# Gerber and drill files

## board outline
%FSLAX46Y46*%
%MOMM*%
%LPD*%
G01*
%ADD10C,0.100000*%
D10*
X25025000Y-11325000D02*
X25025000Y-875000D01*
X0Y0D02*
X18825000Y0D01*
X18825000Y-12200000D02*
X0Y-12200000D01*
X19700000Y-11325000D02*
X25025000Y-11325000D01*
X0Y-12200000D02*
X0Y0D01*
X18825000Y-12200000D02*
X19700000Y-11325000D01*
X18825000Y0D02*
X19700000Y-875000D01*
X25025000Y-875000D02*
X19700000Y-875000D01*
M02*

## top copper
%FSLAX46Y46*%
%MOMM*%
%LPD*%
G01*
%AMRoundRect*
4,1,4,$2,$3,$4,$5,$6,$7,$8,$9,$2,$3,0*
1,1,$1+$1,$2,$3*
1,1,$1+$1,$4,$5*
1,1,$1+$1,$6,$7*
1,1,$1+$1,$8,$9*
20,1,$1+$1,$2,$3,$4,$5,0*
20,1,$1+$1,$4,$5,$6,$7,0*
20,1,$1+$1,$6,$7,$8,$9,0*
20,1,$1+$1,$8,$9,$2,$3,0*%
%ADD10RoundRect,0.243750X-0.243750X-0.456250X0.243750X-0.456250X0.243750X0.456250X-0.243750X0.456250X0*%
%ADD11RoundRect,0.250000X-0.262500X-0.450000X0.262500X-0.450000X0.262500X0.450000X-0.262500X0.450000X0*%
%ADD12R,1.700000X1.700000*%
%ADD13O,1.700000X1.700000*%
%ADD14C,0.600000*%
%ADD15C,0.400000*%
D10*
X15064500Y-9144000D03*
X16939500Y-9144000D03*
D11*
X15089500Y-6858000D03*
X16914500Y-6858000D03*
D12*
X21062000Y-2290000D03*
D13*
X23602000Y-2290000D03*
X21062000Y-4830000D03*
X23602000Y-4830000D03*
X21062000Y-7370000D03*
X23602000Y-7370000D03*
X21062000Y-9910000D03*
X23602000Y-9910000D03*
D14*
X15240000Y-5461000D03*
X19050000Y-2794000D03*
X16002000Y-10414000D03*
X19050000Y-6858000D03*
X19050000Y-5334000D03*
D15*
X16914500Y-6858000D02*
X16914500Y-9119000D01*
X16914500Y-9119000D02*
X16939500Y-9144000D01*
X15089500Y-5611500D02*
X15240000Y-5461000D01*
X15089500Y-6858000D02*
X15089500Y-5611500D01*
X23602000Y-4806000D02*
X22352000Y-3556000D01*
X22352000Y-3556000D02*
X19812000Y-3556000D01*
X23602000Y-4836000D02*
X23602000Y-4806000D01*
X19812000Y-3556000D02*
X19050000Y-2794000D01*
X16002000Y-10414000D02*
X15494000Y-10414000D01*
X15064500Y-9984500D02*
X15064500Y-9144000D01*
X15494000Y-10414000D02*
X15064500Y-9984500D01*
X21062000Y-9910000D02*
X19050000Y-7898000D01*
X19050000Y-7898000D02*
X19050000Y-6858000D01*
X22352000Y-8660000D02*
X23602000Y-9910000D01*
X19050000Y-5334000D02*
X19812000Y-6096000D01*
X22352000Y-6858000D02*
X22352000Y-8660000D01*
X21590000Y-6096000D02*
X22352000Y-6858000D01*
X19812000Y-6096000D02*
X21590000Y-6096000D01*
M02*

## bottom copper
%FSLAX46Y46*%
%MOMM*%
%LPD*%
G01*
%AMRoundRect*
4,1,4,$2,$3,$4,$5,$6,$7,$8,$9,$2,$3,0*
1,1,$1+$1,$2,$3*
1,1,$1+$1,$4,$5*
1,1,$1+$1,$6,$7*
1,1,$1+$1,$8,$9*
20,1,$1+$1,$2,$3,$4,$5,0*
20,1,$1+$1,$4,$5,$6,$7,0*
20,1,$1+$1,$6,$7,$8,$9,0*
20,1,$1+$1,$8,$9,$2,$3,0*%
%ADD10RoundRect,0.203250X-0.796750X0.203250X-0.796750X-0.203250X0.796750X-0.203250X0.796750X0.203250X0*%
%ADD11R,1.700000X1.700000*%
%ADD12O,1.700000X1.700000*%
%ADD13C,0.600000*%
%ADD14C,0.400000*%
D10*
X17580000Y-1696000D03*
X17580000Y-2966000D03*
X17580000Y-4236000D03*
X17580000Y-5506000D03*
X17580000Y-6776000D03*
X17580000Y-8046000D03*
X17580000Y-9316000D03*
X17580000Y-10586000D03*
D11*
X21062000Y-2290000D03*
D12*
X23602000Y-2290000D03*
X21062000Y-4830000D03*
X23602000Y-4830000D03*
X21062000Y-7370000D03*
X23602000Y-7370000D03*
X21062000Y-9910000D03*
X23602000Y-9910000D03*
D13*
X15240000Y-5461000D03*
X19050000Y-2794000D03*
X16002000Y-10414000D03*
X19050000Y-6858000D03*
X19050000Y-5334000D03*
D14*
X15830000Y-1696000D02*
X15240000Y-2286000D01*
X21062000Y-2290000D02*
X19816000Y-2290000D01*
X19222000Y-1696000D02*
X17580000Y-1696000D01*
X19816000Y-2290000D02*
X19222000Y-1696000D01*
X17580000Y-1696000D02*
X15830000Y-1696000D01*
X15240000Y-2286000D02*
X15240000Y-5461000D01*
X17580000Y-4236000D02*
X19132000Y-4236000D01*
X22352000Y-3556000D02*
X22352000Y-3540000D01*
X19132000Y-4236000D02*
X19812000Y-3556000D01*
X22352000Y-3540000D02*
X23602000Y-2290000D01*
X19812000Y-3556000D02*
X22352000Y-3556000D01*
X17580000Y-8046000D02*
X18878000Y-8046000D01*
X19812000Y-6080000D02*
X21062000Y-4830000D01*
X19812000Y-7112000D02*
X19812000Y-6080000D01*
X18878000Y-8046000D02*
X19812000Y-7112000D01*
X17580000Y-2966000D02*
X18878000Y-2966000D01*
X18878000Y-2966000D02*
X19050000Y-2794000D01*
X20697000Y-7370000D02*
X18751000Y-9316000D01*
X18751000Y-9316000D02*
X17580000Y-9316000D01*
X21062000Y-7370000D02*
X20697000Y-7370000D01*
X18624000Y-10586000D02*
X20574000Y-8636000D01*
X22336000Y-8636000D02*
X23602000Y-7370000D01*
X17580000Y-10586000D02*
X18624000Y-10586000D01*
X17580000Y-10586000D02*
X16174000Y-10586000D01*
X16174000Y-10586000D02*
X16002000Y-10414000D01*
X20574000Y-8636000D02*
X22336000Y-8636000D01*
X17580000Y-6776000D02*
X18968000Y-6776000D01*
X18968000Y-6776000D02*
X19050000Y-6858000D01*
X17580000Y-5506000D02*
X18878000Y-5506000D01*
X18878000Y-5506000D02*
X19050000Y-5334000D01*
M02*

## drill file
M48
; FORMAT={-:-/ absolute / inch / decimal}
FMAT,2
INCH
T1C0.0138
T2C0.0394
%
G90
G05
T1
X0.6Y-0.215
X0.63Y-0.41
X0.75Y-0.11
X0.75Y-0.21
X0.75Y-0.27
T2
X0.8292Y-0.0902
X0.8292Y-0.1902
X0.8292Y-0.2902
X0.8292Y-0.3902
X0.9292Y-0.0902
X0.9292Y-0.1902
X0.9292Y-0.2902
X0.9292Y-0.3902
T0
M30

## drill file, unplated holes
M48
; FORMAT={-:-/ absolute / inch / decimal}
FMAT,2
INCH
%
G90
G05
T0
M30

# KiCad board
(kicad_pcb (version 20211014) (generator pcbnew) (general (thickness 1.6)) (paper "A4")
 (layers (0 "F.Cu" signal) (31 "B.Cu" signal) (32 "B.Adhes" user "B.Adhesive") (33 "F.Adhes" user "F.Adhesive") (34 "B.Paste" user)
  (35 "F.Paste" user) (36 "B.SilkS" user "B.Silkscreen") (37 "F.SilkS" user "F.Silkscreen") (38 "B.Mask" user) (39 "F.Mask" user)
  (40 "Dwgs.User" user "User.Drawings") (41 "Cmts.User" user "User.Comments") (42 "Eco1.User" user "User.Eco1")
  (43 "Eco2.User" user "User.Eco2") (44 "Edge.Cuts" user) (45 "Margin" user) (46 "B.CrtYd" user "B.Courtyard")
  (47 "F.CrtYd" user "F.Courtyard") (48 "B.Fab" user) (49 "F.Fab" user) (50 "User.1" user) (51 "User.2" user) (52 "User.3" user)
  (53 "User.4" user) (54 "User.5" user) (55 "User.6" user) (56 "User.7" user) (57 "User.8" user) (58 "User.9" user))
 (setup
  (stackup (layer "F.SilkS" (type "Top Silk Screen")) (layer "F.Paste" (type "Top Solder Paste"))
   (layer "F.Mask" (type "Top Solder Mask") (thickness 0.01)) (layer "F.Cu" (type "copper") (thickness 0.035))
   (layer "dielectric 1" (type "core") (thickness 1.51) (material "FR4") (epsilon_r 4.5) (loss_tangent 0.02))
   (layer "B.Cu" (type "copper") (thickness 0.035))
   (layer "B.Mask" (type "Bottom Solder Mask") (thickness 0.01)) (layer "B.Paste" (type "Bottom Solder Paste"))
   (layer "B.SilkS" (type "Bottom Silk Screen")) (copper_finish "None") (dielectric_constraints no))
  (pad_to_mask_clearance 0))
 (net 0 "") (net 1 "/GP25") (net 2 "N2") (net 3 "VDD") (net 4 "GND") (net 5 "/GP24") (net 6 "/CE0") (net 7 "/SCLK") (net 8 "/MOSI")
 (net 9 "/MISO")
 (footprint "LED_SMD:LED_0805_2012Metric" (layer "F.Cu") (at 16.002 9.144)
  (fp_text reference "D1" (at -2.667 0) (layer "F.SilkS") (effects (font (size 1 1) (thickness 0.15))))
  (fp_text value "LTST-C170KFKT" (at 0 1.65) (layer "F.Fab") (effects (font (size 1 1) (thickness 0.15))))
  (pad "1" smd roundrect (at -0.9375 0) (size 0.975 1.4) (layers "F.Cu" "F.Paste" "F.Mask") (roundrect_rratio 0.25) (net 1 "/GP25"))
  (pad "2" smd roundrect (at 0.9375 0) (size 0.975 1.4) (layers "F.Cu" "F.Paste" "F.Mask") (roundrect_rratio 0.25) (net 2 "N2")))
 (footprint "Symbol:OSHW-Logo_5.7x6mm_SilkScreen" (layer "F.Cu") (at 9.144 8.382)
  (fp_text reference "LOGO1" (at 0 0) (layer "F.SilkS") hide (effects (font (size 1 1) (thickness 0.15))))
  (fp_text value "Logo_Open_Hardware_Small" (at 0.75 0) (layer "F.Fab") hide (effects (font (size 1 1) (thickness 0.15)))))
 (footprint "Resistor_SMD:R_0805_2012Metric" (layer "F.Cu") (at 16.002 6.858)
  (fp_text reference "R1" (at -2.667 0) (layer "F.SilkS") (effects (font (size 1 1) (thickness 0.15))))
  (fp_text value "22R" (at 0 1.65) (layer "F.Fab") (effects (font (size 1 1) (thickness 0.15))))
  (pad "1" smd roundrect (at -0.9125 0) (size 1.025 1.4) (layers "F.Cu" "F.Paste" "F.Mask") (roundrect_rratio 0.243902439) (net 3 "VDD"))
  (pad "2" smd roundrect (at 0.9125 0) (size 1.025 1.4) (layers "F.Cu" "F.Paste" "F.Mask") (roundrect_rratio 0.243902439) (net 2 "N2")))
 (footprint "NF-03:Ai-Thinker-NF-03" (layer "B.Cu") (at 18.08 1.696 -90)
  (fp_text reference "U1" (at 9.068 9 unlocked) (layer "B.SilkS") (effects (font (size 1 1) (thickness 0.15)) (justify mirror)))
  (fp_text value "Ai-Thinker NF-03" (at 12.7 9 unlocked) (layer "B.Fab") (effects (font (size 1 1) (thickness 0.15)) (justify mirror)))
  (pad "1" smd roundrect (at 0 0.5 270) (size 0.813 2) (layers "B.Cu" "B.Paste" "B.Mask") (roundrect_rratio 0.25) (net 3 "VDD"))
  (pad "2" smd roundrect (at 1.27 0.5 270) (size 0.813 2) (layers "B.Cu" "B.Paste" "B.Mask") (roundrect_rratio 0.25) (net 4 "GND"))
  (pad "3" smd roundrect (at 2.54 0.5 270) (size 0.813 2) (layers "B.Cu" "B.Paste" "B.Mask") (roundrect_rratio 0.25) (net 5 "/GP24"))
  (pad "4" smd roundrect (at 3.81 0.5 270) (size 0.813 2) (layers "B.Cu" "B.Paste" "B.Mask") (roundrect_rratio 0.25) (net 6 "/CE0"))
  (pad "5" smd roundrect (at 5.08 0.5 270) (size 0.813 2) (layers "B.Cu" "B.Paste" "B.Mask") (roundrect_rratio 0.25) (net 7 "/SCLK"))
  (pad "6" smd roundrect (at 6.35 0.5 270) (size 0.813 2) (layers "B.Cu" "B.Paste" "B.Mask") (roundrect_rratio 0.25) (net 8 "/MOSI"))
  (pad "7" smd roundrect (at 7.62 0.5 270) (size 0.813 2) (layers "B.Cu" "B.Paste" "B.Mask") (roundrect_rratio 0.25) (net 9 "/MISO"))
  (pad "8" smd roundrect (at 8.89 0.5 270) (size 0.813 2) (layers "B.Cu" "B.Paste" "B.Mask") (roundrect_rratio 0.25) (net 1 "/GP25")))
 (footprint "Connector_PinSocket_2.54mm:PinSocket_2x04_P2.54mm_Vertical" (layer "B.Cu") (at 21.062 2.29 180)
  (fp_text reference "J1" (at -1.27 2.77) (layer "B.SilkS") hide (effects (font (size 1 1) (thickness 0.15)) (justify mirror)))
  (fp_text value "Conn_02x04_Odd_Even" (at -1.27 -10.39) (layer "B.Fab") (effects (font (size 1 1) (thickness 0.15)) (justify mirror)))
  (pad "1" thru_hole rect (at 0 0 180) (size 1.7 1.7) (drill 1) (layers *.Cu *.Mask) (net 3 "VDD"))
  (pad "2" thru_hole oval (at -2.54 0 180) (size 1.7 1.7) (drill 1) (layers *.Cu *.Mask) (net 5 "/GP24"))
  (pad "3" thru_hole oval (at 0 -2.54 180) (size 1.7 1.7) (drill 1) (layers *.Cu *.Mask) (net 8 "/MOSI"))
  (pad "4" thru_hole oval (at -2.54 -2.54 180) (size 1.7 1.7) (drill 1) (layers *.Cu *.Mask) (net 4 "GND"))
  (pad "5" thru_hole oval (at 0 -5.08 180) (size 1.7 1.7) (drill 1) (layers *.Cu *.Mask) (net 9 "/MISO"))
  (pad "6" thru_hole oval (at -2.54 -5.08 180) (size 1.7 1.7) (drill 1) (layers *.Cu *.Mask) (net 1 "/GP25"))
  (pad "7" thru_hole oval (at 0 -7.62 180) (size 1.7 1.7) (drill 1) (layers *.Cu *.Mask) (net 7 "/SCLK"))
  (pad "8" thru_hole oval (at -2.54 -7.62 180) (size 1.7 1.7) (drill 1) (layers *.Cu *.Mask) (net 6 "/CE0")))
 (gr_line (start 25.025 11.325) (end 25.025 0.875) (layer "Edge.Cuts") (width 0.1))
 (gr_line (start 0 0) (end 18.825 0) (layer "Edge.Cuts") (width 0.1))
 (gr_line (start 18.825 12.2) (end 0 12.2) (layer "Edge.Cuts") (width 0.1))
 (gr_line (start 19.7 11.325) (end 25.025 11.325) (layer "Edge.Cuts") (width 0.1))
 (gr_line (start 0 12.2) (end 0 0) (layer "Edge.Cuts") (width 0.1))
 (gr_line (start 18.825 12.2) (end 19.7 11.325) (layer "Edge.Cuts") (width 0.1))
 (gr_line (start 18.825 0) (end 19.7 0.875) (layer "Edge.Cuts") (width 0.1))
 (gr_line (start 25.025 0.875) (end 19.7 0.875) (layer "Edge.Cuts") (width 0.1))
 (segment (start 16.9145 6.858) (end 16.9145 9.119) (width 0.4) (layer "F.Cu") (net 2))
 (segment (start 16.9145 9.119) (end 16.9395 9.144) (width 0.4) (layer "F.Cu") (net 2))
 (segment (start 15.0895 5.6115) (end 15.24 5.461) (width 0.4) (layer "F.Cu") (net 3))
 (segment (start 15.0895 6.858) (end 15.0895 5.6115) (width 0.4) (layer "F.Cu") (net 3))
 (via (at 15.24 5.461) (size 0.6) (drill 0.35) (layers "F.Cu" "B.Cu") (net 3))
 (segment (start 15.83 1.696) (end 15.24 2.286) (width 0.4) (layer "B.Cu") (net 3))
 (segment (start 21.062 2.29) (end 19.816 2.29) (width 0.4) (layer "B.Cu") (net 3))
 (segment (start 19.222 1.696) (end 17.58 1.696) (width 0.4) (layer "B.Cu") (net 3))
 (segment (start 19.816 2.29) (end 19.222 1.696) (width 0.4) (layer "B.Cu") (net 3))
 (segment (start 17.58 1.696) (end 15.83 1.696) (width 0.4) (layer "B.Cu") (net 3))
 (segment (start 15.24 2.286) (end 15.24 5.461) (width 0.4) (layer "B.Cu") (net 3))
 (segment (start 17.58 4.236) (end 19.132 4.236) (width 0.4) (layer "B.Cu") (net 5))
 (segment (start 22.352 3.556) (end 22.352 3.54) (width 0.4) (layer "B.Cu") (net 5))
 (segment (start 19.132 4.236) (end 19.812 3.556) (width 0.4) (layer "B.Cu") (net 5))
 (segment (start 22.352 3.54) (end 23.602 2.29) (width 0.4) (layer "B.Cu") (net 5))
 (segment (start 19.812 3.556) (end 22.352 3.556) (width 0.4) (layer "B.Cu") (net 5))
 (segment (start 17.58 8.046) (end 18.878 8.046) (width 0.4) (layer "B.Cu") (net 8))
 (segment (start 19.812 6.08) (end 21.062 4.83) (width 0.4) (layer "B.Cu") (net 8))
 (segment (start 19.812 7.112) (end 19.812 6.08) (width 0.4) (layer "B.Cu") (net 8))
 (segment (start 18.878 8.046) (end 19.812 7.112) (width 0.4) (layer "B.Cu") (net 8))
 (segment (start 23.602 4.806) (end 22.352 3.556) (width 0.4) (layer "F.Cu") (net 4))
 (segment (start 22.352 3.556) (end 19.812 3.556) (width 0.4) (layer "F.Cu") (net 4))
 (segment (start 23.602 4.836) (end 23.602 4.806) (width 0.4) (layer "F.Cu") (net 4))
 (segment (start 19.812 3.556) (end 19.05 2.794) (width 0.4) (layer "F.Cu") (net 4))
 (via (at 19.05 2.794) (size 0.6) (drill 0.35) (layers "F.Cu" "B.Cu") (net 4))
 (segment (start 17.58 2.966) (end 18.878 2.966) (width 0.4) (layer "B.Cu") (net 4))
 (segment (start 18.878 2.966) (end 19.05 2.794) (width 0.4) (layer "B.Cu") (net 4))
 (segment (start 20.697 7.37) (end 18.751 9.316) (width 0.4) (layer "B.Cu") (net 9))
 (segment (start 18.751 9.316) (end 17.58 9.316) (width 0.4) (layer "B.Cu") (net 9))
 (segment (start 21.062 7.37) (end 20.697 7.37) (width 0.4) (layer "B.Cu") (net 9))
 (segment (start 16.002 10.414) (end 15.494 10.414) (width 0.4) (layer "F.Cu") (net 1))
 (segment (start 15.0645 9.9845) (end 15.0645 9.144) (width 0.4) (layer "F.Cu") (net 1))
 (segment (start 15.494 10.414) (end 15.0645 9.9845) (width 0.4) (layer "F.Cu") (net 1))
 (via (at 16.002 10.414) (size 0.6) (drill 0.35) (layers "F.Cu" "B.Cu") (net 1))
 (segment (start 18.624 10.586) (end 20.574 8.636) (width 0.4) (layer "B.Cu") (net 1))
 (segment (start 22.336 8.636) (end 23.602 7.37) (width 0.4) (layer "B.Cu") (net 1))
 (segment (start 17.58 10.586) (end 18.624 10.586) (width 0.4) (layer "B.Cu") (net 1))
 (segment (start 17.58 10.586) (end 16.174 10.586) (width 0.4) (layer "B.Cu") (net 1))
 (segment (start 16.174 10.586) (end 16.002 10.414) (width 0.4) (layer "B.Cu") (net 1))
 (segment (start 20.574 8.636) (end 22.336 8.636) (width 0.4) (layer "B.Cu") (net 1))
 (segment (start 21.062 9.91) (end 19.05 7.898) (width 0.4) (layer "F.Cu") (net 7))
 (segment (start 19.05 7.898) (end 19.05 6.858) (width 0.4) (layer "F.Cu") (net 7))
 (via (at 19.05 6.858) (size 0.6) (drill 0.35) (layers "F.Cu" "B.Cu") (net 7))
 (segment (start 17.58 6.776) (end 18.968 6.776) (width 0.4) (layer "B.Cu") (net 7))
 (segment (start 18.968 6.776) (end 19.05 6.858) (width 0.4) (layer "B.Cu") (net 7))
 (segment (start 22.352 8.66) (end 23.602 9.91) (width 0.4) (layer "F.Cu") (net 6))
 (segment (start 19.05 5.334) (end 19.812 6.096) (width 0.4) (layer "F.Cu") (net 6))
 (segment (start 22.352 6.858) (end 22.352 8.66) (width 0.4) (layer "F.Cu") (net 6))
 (segment (start 21.59 6.096) (end 22.352 6.858) (width 0.4) (layer "F.Cu") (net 6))
 (segment (start 19.812 6.096) (end 21.59 6.096) (width 0.4) (layer "F.Cu") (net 6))
 (via (at 19.05 5.334) (size 0.6) (drill 0.35) (layers "F.Cu" "B.Cu") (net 6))
 (segment (start 17.58 5.506) (end 18.878 5.506) (width 0.4) (layer "B.Cu") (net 6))
 (segment (start 18.878 5.506) (end 19.05 5.334) (width 0.4) (layer "B.Cu") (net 6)))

